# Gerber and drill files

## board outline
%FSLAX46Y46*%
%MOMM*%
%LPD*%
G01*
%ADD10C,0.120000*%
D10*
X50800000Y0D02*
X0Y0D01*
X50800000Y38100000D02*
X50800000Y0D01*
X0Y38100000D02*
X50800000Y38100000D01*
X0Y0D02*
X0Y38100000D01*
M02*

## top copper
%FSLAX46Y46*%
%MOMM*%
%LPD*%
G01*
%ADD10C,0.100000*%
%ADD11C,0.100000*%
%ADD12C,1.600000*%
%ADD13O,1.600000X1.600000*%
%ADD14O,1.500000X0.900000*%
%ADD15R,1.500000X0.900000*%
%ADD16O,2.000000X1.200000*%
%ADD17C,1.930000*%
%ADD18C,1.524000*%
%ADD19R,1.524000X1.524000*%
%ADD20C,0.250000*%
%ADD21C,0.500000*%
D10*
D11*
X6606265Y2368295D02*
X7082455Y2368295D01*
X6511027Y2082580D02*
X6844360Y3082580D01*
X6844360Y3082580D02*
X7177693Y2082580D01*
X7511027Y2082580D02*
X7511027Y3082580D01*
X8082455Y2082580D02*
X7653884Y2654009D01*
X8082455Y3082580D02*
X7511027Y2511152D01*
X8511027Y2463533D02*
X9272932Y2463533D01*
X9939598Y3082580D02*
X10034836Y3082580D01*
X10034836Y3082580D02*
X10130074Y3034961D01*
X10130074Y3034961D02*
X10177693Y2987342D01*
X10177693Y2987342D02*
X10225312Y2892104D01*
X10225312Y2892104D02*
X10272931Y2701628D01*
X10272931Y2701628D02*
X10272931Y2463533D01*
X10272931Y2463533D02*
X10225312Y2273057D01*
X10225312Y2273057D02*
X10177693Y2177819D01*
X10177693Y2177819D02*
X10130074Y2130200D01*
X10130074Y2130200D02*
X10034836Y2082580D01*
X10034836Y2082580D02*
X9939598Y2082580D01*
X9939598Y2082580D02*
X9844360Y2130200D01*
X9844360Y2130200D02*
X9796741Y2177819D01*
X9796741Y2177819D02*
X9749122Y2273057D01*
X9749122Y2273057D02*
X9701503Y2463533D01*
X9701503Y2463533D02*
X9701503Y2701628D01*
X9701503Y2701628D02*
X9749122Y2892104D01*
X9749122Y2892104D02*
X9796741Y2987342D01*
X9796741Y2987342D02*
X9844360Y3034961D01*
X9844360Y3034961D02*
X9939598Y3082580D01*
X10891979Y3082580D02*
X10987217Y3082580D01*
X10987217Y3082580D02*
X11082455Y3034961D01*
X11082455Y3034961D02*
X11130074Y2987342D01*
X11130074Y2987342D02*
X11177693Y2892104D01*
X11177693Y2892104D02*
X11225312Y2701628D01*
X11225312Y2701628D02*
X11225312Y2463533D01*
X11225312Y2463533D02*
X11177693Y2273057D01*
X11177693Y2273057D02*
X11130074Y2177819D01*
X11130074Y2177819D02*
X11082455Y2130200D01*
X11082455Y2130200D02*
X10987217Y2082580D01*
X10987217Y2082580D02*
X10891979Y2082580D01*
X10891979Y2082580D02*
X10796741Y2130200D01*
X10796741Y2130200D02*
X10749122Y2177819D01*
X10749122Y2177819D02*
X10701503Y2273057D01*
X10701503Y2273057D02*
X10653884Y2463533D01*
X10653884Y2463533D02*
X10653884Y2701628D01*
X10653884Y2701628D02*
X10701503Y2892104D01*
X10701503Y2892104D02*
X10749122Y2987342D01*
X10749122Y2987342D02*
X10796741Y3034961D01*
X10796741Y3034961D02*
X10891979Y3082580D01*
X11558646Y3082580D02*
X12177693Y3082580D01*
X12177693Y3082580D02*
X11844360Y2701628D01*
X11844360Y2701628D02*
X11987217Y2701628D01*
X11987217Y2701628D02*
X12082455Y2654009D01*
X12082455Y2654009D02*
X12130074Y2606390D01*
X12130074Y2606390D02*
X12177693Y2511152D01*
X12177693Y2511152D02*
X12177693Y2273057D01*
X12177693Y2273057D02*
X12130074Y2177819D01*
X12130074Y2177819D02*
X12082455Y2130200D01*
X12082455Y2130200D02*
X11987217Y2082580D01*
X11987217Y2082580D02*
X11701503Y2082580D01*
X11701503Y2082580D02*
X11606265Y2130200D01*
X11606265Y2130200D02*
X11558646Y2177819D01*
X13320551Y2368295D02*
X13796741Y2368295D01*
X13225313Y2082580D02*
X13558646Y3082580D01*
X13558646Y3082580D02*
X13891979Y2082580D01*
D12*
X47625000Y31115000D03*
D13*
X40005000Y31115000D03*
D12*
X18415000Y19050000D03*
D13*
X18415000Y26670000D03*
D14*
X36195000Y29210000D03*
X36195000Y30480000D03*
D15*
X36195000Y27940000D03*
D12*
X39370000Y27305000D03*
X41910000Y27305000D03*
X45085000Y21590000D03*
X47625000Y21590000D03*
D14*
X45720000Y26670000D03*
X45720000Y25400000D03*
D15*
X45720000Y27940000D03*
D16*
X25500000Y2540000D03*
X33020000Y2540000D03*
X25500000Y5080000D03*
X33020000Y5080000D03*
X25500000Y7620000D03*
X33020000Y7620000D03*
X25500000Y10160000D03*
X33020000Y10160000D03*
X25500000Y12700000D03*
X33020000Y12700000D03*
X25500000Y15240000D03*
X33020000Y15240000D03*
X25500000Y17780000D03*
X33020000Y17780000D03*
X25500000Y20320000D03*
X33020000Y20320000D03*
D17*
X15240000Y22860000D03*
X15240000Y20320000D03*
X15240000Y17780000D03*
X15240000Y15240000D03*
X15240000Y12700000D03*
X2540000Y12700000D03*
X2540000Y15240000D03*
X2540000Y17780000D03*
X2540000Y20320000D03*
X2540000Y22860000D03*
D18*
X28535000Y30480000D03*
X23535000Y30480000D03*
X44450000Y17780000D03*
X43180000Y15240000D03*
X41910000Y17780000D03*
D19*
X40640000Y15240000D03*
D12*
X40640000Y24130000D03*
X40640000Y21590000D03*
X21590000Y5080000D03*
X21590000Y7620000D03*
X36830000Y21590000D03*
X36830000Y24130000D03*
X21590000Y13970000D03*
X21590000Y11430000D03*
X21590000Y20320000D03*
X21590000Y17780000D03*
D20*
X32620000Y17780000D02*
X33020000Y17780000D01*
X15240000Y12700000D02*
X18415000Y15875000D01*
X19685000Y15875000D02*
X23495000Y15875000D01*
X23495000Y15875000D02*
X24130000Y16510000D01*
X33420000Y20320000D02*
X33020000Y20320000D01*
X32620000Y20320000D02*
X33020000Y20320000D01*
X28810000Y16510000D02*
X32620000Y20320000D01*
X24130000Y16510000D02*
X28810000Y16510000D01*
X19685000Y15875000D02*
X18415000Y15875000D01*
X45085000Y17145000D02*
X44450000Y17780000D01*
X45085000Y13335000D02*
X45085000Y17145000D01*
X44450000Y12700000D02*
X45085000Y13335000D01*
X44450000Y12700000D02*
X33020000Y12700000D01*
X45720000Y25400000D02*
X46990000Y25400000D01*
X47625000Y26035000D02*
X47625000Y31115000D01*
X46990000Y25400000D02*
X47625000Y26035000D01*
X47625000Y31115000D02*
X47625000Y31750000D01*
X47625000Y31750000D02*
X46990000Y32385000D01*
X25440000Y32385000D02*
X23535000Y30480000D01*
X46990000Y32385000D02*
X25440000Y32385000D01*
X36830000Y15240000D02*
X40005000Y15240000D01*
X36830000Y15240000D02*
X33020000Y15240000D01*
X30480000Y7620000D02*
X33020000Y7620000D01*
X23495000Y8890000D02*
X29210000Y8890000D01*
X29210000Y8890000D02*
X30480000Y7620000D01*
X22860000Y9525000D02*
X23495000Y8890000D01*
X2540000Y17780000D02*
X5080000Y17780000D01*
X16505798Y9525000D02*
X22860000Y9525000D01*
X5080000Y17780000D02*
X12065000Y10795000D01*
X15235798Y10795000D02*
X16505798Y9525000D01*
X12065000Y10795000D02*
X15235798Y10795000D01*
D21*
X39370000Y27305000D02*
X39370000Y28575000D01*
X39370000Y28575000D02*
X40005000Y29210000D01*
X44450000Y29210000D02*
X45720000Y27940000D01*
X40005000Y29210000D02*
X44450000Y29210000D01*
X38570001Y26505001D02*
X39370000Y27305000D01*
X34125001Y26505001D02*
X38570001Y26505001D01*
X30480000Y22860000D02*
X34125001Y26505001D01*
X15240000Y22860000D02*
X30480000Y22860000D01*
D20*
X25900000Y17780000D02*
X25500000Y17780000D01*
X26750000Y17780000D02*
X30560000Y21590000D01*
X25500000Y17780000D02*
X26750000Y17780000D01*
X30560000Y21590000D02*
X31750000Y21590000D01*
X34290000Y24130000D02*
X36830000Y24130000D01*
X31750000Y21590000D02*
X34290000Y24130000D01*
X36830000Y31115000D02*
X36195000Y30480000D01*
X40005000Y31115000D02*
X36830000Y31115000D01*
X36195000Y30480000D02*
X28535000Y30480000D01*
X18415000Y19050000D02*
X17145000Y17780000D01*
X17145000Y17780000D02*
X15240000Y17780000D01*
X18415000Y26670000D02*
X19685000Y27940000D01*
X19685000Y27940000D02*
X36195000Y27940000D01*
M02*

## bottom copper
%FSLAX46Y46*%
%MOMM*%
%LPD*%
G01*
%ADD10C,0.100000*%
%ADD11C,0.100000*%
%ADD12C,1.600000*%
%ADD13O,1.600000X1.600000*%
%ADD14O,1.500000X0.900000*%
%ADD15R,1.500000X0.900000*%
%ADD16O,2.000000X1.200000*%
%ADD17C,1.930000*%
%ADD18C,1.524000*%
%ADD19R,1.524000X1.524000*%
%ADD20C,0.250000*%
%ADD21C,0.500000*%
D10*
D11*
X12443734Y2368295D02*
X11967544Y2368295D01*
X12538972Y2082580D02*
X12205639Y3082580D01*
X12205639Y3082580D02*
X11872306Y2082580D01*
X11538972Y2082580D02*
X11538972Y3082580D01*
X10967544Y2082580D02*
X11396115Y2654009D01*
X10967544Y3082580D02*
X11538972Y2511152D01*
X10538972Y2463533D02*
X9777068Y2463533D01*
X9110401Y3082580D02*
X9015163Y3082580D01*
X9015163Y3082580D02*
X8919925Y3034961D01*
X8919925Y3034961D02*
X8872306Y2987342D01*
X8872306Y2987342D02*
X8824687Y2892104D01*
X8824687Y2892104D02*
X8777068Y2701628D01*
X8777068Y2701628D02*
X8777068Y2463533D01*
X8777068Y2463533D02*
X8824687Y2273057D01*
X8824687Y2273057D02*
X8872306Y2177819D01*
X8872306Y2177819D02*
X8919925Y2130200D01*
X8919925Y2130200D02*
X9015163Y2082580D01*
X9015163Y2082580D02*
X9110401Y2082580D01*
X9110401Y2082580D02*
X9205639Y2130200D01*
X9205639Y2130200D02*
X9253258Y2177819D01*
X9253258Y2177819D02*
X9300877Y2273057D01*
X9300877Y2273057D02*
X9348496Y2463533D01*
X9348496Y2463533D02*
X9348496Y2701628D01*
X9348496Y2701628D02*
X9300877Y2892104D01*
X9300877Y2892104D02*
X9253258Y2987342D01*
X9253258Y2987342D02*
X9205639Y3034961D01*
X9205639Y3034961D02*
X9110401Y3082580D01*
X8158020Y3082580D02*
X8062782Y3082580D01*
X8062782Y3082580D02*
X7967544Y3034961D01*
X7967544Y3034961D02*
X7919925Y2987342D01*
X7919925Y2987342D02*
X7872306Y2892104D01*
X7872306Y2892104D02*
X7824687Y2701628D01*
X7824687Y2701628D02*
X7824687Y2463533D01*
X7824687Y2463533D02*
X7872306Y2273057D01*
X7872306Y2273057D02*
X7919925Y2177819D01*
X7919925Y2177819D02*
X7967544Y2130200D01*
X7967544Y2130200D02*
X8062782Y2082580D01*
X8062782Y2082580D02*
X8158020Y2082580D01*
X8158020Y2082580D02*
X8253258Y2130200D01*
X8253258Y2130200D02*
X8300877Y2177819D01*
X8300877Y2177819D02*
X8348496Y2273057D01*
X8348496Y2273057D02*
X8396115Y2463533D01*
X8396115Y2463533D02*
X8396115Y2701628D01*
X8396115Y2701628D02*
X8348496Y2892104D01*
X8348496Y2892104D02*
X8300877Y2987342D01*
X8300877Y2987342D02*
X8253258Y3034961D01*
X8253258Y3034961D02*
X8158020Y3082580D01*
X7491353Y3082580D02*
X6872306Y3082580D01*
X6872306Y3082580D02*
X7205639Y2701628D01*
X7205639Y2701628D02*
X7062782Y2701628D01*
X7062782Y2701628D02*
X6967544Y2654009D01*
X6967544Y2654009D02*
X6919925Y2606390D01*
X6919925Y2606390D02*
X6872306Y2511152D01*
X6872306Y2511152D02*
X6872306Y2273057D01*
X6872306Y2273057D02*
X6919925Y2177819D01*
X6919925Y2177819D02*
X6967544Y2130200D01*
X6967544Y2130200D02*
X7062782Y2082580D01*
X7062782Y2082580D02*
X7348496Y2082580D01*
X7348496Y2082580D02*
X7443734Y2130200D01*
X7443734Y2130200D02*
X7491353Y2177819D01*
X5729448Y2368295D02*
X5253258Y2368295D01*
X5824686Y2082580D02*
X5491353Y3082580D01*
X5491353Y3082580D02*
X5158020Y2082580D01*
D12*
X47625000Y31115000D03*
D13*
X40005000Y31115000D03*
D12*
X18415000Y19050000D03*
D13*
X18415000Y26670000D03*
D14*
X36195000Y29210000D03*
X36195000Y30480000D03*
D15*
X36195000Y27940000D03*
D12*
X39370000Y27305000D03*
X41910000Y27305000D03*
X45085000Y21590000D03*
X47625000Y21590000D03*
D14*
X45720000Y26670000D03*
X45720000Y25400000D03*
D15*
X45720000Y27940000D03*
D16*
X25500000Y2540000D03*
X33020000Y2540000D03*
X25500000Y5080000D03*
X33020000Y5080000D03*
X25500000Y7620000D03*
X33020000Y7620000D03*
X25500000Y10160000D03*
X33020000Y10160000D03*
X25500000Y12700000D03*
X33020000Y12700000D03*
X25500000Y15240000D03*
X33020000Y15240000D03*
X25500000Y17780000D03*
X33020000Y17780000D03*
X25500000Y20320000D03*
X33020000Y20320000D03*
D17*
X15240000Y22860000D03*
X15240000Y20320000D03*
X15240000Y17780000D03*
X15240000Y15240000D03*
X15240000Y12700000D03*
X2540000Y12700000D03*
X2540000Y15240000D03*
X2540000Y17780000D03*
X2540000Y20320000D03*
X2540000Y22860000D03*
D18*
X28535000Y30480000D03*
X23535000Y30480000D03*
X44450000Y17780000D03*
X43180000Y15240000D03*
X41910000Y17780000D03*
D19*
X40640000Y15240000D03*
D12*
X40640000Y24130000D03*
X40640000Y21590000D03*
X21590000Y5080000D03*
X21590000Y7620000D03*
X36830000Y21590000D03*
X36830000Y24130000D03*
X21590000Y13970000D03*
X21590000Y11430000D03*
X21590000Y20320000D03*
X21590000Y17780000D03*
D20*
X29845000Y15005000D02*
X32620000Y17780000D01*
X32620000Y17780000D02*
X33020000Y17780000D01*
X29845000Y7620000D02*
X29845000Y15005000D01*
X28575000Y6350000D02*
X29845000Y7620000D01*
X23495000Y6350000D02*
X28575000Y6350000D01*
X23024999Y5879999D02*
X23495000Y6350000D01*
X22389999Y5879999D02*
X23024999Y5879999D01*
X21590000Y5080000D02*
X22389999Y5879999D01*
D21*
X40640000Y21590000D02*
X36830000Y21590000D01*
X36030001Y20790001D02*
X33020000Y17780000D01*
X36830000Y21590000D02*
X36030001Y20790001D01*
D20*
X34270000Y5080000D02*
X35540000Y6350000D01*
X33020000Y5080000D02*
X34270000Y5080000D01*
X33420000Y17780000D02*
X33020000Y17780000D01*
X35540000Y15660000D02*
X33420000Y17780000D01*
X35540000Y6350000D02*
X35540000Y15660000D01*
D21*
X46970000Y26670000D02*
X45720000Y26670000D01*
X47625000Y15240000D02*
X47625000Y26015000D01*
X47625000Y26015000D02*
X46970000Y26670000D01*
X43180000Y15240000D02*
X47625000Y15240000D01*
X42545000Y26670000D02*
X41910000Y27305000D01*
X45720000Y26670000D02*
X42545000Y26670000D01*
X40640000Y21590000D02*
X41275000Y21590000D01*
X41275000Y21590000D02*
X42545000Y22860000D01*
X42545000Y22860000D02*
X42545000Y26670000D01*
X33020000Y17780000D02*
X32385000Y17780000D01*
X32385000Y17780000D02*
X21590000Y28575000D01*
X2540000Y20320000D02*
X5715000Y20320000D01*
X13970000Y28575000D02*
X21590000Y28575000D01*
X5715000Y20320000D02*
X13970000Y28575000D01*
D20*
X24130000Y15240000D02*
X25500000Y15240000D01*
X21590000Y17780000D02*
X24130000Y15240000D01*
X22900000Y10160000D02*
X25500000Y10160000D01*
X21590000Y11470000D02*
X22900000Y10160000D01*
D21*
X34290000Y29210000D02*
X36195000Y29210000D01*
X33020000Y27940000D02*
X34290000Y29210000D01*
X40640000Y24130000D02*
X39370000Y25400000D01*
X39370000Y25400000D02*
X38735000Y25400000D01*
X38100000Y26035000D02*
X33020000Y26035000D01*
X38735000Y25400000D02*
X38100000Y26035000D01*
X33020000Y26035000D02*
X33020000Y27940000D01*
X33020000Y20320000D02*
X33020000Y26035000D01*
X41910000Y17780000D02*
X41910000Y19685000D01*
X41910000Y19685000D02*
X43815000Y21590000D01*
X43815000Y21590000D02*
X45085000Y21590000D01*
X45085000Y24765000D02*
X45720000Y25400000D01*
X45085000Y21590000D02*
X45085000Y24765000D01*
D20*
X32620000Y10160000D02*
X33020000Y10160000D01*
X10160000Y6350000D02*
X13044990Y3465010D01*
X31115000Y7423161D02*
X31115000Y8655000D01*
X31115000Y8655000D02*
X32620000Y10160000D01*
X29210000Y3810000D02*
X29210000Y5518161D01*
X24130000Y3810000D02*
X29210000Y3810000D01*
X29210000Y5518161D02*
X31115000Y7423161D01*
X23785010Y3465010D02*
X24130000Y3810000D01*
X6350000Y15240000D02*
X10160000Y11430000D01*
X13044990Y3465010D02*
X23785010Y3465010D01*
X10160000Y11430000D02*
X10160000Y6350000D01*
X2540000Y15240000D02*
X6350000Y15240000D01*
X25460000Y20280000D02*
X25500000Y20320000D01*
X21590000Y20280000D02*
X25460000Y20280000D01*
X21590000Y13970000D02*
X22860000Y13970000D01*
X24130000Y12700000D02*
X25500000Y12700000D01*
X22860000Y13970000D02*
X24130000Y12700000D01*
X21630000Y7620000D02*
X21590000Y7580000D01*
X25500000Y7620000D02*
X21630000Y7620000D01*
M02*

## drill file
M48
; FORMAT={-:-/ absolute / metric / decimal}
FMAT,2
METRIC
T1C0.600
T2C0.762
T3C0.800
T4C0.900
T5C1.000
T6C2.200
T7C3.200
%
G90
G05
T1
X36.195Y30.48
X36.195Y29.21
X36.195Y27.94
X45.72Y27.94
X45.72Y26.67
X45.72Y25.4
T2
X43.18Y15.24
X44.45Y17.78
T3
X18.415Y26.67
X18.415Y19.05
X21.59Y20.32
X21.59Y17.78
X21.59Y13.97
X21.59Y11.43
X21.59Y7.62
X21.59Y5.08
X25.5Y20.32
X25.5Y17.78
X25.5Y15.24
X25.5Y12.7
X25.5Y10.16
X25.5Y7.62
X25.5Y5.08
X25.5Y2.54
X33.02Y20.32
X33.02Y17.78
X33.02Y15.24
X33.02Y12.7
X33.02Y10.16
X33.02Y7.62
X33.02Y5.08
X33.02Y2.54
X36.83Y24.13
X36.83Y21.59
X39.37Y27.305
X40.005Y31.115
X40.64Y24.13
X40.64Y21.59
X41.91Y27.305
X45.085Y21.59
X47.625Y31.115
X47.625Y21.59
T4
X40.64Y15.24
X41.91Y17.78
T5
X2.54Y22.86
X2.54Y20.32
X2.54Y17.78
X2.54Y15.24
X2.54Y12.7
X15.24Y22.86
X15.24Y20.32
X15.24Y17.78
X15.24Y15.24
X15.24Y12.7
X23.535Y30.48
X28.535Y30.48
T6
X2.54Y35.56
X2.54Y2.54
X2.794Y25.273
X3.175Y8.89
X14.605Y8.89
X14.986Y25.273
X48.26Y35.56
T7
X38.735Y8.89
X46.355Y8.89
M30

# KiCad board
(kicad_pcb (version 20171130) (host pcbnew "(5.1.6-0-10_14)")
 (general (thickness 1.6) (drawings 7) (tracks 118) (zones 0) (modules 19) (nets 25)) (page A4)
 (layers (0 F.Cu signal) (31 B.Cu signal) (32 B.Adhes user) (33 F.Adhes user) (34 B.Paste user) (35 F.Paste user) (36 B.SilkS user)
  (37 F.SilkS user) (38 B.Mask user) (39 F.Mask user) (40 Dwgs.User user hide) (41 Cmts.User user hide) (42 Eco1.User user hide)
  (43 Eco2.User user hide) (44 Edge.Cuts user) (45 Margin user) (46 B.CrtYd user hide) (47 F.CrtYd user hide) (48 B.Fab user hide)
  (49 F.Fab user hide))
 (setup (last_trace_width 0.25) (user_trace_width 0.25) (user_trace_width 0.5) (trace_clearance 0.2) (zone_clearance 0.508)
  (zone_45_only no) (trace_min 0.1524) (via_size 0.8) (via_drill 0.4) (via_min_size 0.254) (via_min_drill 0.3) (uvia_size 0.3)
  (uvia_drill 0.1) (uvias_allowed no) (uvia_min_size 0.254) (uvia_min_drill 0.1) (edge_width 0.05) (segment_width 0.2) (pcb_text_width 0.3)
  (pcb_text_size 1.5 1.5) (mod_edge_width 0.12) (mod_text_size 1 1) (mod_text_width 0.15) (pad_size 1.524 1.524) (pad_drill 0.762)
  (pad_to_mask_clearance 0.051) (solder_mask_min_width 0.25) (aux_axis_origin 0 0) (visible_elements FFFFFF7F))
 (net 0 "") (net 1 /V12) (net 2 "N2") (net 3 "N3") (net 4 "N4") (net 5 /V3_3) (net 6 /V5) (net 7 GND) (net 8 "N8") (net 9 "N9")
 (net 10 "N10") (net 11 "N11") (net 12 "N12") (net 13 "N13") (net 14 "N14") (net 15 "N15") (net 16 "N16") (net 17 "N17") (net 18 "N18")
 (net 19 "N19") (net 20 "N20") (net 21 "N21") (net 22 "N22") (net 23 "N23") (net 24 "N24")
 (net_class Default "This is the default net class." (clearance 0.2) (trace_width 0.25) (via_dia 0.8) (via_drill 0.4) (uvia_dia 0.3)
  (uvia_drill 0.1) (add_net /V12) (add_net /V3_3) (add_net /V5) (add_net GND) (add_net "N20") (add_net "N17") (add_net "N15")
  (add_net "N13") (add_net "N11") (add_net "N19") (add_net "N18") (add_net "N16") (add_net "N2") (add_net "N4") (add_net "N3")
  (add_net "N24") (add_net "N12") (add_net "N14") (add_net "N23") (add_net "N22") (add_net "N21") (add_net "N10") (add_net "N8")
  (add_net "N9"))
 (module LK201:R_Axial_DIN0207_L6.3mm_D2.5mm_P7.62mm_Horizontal (layer F.Cu) (at 47.625 -31.115 180)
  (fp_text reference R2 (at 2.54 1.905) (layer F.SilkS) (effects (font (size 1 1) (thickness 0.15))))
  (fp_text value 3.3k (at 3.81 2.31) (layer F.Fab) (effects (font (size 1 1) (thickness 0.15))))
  (pad 1 thru_hole circle (at 0 0 180) (size 1.6 1.6) (drill 0.8) (layers *.Cu *.Mask) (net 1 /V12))
  (pad 2 thru_hole oval (at 7.62 0 180) (size 1.6 1.6) (drill 0.8) (layers *.Cu *.Mask) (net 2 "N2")))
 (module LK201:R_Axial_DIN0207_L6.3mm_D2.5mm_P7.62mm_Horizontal (layer F.Cu) (at 18.415 -19.05 90)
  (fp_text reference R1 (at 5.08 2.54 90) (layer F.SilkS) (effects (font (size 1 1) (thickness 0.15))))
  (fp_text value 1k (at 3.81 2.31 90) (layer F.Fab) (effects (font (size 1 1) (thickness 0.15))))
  (pad 1 thru_hole circle (at 0 0 90) (size 1.6 1.6) (drill 0.8) (layers *.Cu *.Mask) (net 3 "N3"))
  (pad 2 thru_hole oval (at 7.62 0 90) (size 1.6 1.6) (drill 0.8) (layers *.Cu *.Mask) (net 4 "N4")))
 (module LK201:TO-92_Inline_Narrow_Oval (layer F.Cu) (at 36.195 -27.94 90)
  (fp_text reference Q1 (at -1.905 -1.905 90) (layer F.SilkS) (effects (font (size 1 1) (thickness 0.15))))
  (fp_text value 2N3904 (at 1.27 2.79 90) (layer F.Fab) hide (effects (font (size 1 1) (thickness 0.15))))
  (pad 2 thru_hole oval (at 1.27 0 270) (size 0.9 1.5) (drill 0.6) (layers *.Cu *.Mask) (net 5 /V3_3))
  (pad 3 thru_hole oval (at 2.54 0 270) (size 0.9 1.5) (drill 0.6) (layers *.Cu *.Mask) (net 2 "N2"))
  (pad 1 thru_hole rect (at 0 0 270) (size 0.9 1.5) (drill 0.6) (layers *.Cu *.Mask) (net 4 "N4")))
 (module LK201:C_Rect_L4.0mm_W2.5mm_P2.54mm (layer F.Cu) (at 39.37 -27.305)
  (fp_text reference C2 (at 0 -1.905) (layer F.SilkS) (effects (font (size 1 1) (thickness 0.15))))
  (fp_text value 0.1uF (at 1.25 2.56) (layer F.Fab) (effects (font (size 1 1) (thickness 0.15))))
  (pad 1 thru_hole circle (at 0 0) (size 1.6 1.6) (drill 0.8) (layers *.Cu *.Mask) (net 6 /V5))
  (pad 2 thru_hole circle (at 2.54 0) (size 1.6 1.6) (drill 0.8) (layers *.Cu *.Mask) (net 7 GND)))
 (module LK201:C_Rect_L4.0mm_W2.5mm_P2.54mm (layer F.Cu) (at 45.085 -21.59)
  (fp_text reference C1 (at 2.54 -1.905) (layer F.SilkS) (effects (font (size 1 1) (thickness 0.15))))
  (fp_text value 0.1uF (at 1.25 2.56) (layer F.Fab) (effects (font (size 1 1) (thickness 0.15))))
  (pad 1 thru_hole circle (at 0 0) (size 1.6 1.6) (drill 0.8) (layers *.Cu *.Mask) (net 1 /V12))
  (pad 2 thru_hole circle (at 2.54 0) (size 1.6 1.6) (drill 0.8) (layers *.Cu *.Mask) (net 7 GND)))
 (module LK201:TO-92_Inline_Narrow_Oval (layer F.Cu) (at 45.72 -27.94 270)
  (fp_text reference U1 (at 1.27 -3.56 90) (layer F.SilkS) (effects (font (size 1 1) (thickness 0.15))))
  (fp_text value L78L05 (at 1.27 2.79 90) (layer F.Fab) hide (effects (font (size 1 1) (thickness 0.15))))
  (pad 2 thru_hole oval (at 1.27 0 90) (size 0.9 1.5) (drill 0.6) (layers *.Cu *.Mask) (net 7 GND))
  (pad 3 thru_hole oval (at 2.54 0 90) (size 0.9 1.5) (drill 0.6) (layers *.Cu *.Mask) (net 1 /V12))
  (pad 1 thru_hole rect (at 0 0 90) (size 0.9 1.5) (drill 0.6) (layers *.Cu *.Mask) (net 6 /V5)))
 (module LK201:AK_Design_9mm (layer F.Cu) (at 33.655 -33.655)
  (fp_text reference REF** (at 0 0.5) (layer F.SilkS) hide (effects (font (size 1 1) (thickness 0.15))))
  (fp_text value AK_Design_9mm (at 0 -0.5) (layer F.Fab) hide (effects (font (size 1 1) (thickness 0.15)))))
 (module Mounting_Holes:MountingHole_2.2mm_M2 (layer F.Cu) (at 2.54 -2.54)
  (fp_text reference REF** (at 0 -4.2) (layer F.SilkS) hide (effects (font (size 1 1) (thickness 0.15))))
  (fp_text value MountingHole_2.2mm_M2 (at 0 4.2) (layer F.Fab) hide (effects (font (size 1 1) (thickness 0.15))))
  (pad 1 np_thru_hole circle (at 0 0) (size 2.2 2.2) (drill 2.2) (layers *.Cu *.Mask)))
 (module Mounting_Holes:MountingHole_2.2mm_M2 (layer F.Cu) (at 2.54 -35.56)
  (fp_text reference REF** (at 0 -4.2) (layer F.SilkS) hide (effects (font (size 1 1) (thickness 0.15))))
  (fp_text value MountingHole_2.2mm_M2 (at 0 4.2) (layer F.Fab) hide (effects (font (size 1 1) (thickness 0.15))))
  (pad 1 np_thru_hole circle (at 0 0) (size 2.2 2.2) (drill 2.2) (layers *.Cu *.Mask)))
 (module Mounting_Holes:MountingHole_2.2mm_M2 (layer F.Cu) (at 48.26 -35.56)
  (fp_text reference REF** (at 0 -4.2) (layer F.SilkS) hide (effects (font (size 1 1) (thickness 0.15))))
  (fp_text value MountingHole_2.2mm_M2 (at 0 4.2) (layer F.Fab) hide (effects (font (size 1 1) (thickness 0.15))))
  (pad 1 np_thru_hole circle (at 0 0) (size 2.2 2.2) (drill 2.2) (layers *.Cu *.Mask)))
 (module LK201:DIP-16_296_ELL (layer F.Cu) (at 29.26 -11.43 270)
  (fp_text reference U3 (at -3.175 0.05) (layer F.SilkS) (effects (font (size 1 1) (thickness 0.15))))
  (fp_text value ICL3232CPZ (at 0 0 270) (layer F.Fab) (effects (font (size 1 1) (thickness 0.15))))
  (pad 8 thru_hole oval (at 8.89 3.76 270) (size 1.2 2) (drill 0.8) (layers *.Cu *.Mask) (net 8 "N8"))
  (pad 9 thru_hole oval (at 8.89 -3.76 270) (size 1.2 2) (drill 0.8) (layers *.Cu *.Mask) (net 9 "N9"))
  (pad 7 thru_hole oval (at 6.35 3.76 270) (size 1.2 2) (drill 0.8) (layers *.Cu *.Mask) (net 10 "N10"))
  (pad 10 thru_hole oval (at 6.35 -3.76 270) (size 1.2 2) (drill 0.8) (layers *.Cu *.Mask) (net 7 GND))
  (pad 6 thru_hole oval (at 3.81 3.76 270) (size 1.2 2) (drill 0.8) (layers *.Cu *.Mask) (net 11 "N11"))
  (pad 11 thru_hole oval (at 3.81 -3.76 270) (size 1.2 2) (drill 0.8) (layers *.Cu *.Mask) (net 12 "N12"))
  (pad 5 thru_hole oval (at 1.27 3.76 270) (size 1.2 2) (drill 0.8) (layers *.Cu *.Mask) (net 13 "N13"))
  (pad 12 thru_hole oval (at 1.27 -3.76 270) (size 1.2 2) (drill 0.8) (layers *.Cu *.Mask) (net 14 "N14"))
  (pad 4 thru_hole oval (at -1.27 3.76 270) (size 1.2 2) (drill 0.8) (layers *.Cu *.Mask) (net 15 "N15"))
  (pad 13 thru_hole oval (at -1.27 -3.76 270) (size 1.2 2) (drill 0.8) (layers *.Cu *.Mask) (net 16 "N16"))
  (pad 3 thru_hole oval (at -3.81 3.76 270) (size 1.2 2) (drill 0.8) (layers *.Cu *.Mask) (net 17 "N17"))
  (pad 14 thru_hole oval (at -3.81 -3.76 270) (size 1.2 2) (drill 0.8) (layers *.Cu *.Mask) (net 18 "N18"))
  (pad 2 thru_hole oval (at -6.35 3.76 270) (size 1.2 2) (drill 0.8) (layers *.Cu *.Mask) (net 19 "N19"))
  (pad 15 thru_hole oval (at -6.35 -3.76 270) (size 1.2 2) (drill 0.8) (layers *.Cu *.Mask) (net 7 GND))
  (pad 1 thru_hole oval (at -8.89 3.76 270) (size 1.2 2) (drill 0.8) (layers *.Cu *.Mask) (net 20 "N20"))
  (pad 16 thru_hole oval (at -8.89 -3.76 270) (size 1.2 2) (drill 0.8) (layers *.Cu *.Mask) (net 5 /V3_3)))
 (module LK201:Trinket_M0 (layer F.Cu) (at 8.89 -19.05 180)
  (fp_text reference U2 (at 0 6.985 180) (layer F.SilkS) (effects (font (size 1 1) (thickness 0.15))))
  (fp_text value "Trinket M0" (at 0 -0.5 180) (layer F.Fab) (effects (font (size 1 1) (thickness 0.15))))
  (pad 10 thru_hole circle (at -6.35 3.81 180) (size 1.93 1.93) (drill 1) (layers *.Cu *.Mask) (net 6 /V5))
  (pad 9 thru_hole circle (at -6.35 1.27 180) (size 1.93 1.93) (drill 1) (layers *.Cu *.Mask) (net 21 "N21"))
  (pad 8 thru_hole circle (at -6.35 -1.27 180) (size 1.93 1.93) (drill 1) (layers *.Cu *.Mask) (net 3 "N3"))
  (pad 7 thru_hole circle (at -6.35 -3.81 180) (size 1.93 1.93) (drill 1) (layers *.Cu *.Mask) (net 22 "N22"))
  (pad 6 thru_hole circle (at -6.35 -6.35 180) (size 1.93 1.93) (drill 1) (layers *.Cu *.Mask) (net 5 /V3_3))
  (pad 5 thru_hole circle (at 6.35 -6.35 180) (size 1.93 1.93) (drill 1) (layers *.Cu *.Mask) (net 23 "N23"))
  (pad 4 thru_hole circle (at 6.35 -3.81 180) (size 1.93 1.93) (drill 1) (layers *.Cu *.Mask) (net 14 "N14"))
  (pad 3 thru_hole circle (at 6.35 -1.27 180) (size 1.93 1.93) (drill 1) (layers *.Cu *.Mask) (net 12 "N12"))
  (pad 2 thru_hole circle (at 6.35 1.27 180) (size 1.93 1.93) (drill 1) (layers *.Cu *.Mask) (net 7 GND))
  (pad 1 thru_hole circle (at 6.35 3.81 180) (size 1.93 1.93) (drill 1) (layers *.Cu *.Mask) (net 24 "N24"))
  (pad "" np_thru_hole circle (at -5.715 -10.16 180) (size 2.2 2.2) (drill 2.2) (layers *.Mask F.Cu))
  (pad "" np_thru_hole circle (at 5.715 -10.16 180) (size 2.2 2.2) (drill 2.2) (layers *.Mask F.Cu))
  (pad "" np_thru_hole circle (at 6.096 6.223 180) (size 2.2 2.2) (drill 2.2) (layers *.Mask F.Cu))
  (pad "" np_thru_hole circle (at -6.096 6.223 180) (size 2.2 2.2) (drill 2.2) (layers *.Mask F.Cu)))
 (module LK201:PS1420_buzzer (layer F.Cu) (at 26.035 -30.48 180)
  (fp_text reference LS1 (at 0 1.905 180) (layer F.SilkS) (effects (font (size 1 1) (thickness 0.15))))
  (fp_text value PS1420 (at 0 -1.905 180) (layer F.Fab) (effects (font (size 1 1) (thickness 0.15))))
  (pad 2 thru_hole circle (at -2.5 0 180) (size 1.524 1.524) (drill 1) (layers *.Cu *.Mask) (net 2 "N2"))
  (pad 1 thru_hole circle (at 2.5 0 180) (size 1.524 1.524) (drill 1) (layers *.Cu *.Mask) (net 1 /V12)))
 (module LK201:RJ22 (layer F.Cu) (at 42.545 -8.89)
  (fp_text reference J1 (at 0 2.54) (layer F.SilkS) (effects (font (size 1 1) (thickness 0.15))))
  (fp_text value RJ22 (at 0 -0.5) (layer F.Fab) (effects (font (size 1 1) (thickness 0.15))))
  (pad "" np_thru_hole circle (at -3.81 0) (size 3.2 3.2) (drill 3.2) (layers *.Mask F.Cu))
  (pad "" np_thru_hole circle (at 3.81 0) (size 3.2 3.2) (drill 3.2) (layers *.Mask F.Cu))
  (pad 4 thru_hole circle (at 1.905 -8.89) (size 1.524 1.524) (drill 0.762) (layers *.Cu *.Mask) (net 16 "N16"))
  (pad 3 thru_hole circle (at 0.635 -6.35) (size 1.524 1.524) (drill 0.762) (layers *.Cu *.Mask) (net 7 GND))
  (pad 2 thru_hole circle (at -0.635 -8.89) (size 1.524 1.524) (drill 0.9) (layers *.Cu *.Mask) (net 1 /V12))
  (pad 1 thru_hole rect (at -1.905 -6.35) (size 1.524 1.524) (drill 0.9) (layers *.Cu *.Mask) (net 18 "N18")))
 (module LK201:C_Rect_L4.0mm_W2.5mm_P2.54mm (layer F.Cu) (at 40.64 -24.13 270)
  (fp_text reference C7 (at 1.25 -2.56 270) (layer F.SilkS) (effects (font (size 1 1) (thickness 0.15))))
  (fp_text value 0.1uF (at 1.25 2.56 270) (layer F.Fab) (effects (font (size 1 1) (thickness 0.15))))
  (pad 1 thru_hole circle (at 0 0 270) (size 1.6 1.6) (drill 0.8) (layers *.Cu *.Mask) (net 5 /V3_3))
  (pad 2 thru_hole circle (at 2.54 0 270) (size 1.6 1.6) (drill 0.8) (layers *.Cu *.Mask) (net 7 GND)))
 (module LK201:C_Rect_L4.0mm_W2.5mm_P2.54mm (layer F.Cu) (at 21.59 -5.08 90)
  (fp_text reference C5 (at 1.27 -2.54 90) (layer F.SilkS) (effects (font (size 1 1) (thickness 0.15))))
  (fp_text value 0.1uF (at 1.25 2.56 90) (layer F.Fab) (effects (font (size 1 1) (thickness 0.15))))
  (pad 1 thru_hole circle (at 0 0 90) (size 1.6 1.6) (drill 0.8) (layers *.Cu *.Mask) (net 7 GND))
  (pad 2 thru_hole circle (at 2.54 0 90) (size 1.6 1.6) (drill 0.8) (layers *.Cu *.Mask) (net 11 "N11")))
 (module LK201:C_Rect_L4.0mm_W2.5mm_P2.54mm (layer F.Cu) (at 36.83 -21.59 90)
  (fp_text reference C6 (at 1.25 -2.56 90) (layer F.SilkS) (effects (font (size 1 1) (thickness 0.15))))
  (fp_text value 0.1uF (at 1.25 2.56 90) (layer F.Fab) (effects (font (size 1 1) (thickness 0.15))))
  (pad 1 thru_hole circle (at 0 0 90) (size 1.6 1.6) (drill 0.8) (layers *.Cu *.Mask) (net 7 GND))
  (pad 2 thru_hole circle (at 2.54 0 90) (size 1.6 1.6) (drill 0.8) (layers *.Cu *.Mask) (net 19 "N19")))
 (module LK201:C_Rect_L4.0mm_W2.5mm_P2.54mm (layer F.Cu) (at 21.59 -13.97 270)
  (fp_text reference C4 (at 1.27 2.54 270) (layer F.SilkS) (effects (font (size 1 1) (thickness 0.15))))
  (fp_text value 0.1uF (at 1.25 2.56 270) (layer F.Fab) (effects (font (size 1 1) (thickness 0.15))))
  (pad 1 thru_hole circle (at 0 0 270) (size 1.6 1.6) (drill 0.8) (layers *.Cu *.Mask) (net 15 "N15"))
  (pad 2 thru_hole circle (at 2.54 0 270) (size 1.6 1.6) (drill 0.8) (layers *.Cu *.Mask) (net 13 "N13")))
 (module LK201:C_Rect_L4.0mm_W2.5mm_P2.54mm (layer F.Cu) (at 21.59 -20.32 270)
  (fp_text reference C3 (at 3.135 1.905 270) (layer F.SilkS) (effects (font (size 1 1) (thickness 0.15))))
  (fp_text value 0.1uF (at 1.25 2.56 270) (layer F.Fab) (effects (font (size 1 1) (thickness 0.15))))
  (pad 1 thru_hole circle (at 0 0 270) (size 1.6 1.6) (drill 0.8) (layers *.Cu *.Mask) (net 20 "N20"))
  (pad 2 thru_hole circle (at 2.54 0 270) (size 1.6 1.6) (drill 0.8) (layers *.Cu *.Mask) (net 17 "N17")))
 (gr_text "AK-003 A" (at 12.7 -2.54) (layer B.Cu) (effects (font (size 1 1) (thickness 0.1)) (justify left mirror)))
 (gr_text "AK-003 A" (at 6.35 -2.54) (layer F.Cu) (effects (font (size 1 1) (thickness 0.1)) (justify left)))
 (gr_line (start 50.8 0) (end 0 0) (layer Edge.Cuts) (width 0.12))
 (gr_line (start 50.8 -38.1) (end 50.8 0) (layer Edge.Cuts) (width 0.12))
 (gr_line (start 0 -38.1) (end 50.8 -38.1) (layer Edge.Cuts) (width 0.12))
 (gr_line (start 0 0) (end 0 -38.1) (layer Edge.Cuts) (width 0.12))
 (segment (start 29.845 -15.005) (end 32.62 -17.78) (width 0.25) (layer B.Cu) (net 7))
 (segment (start 32.62 -17.78) (end 33.02 -17.78) (width 0.25) (layer B.Cu) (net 7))
 (segment (start 29.845 -7.62) (end 29.845 -15.005) (width 0.25) (layer B.Cu) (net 7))
 (segment (start 28.575 -6.35) (end 29.845 -7.62) (width 0.25) (layer B.Cu) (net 7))
 (segment (start 23.495 -6.35) (end 28.575 -6.35) (width 0.25) (layer B.Cu) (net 7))
 (segment (start 23.024999 -5.879999) (end 23.495 -6.35) (width 0.25) (layer B.Cu) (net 7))
 (segment (start 22.389999 -5.879999) (end 23.024999 -5.879999) (width 0.25) (layer B.Cu) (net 7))
 (segment (start 21.59 -5.08) (end 22.389999 -5.879999) (width 0.25) (layer B.Cu) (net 7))
 (segment (start 32.62 -17.78) (end 33.02 -17.78) (width 0.25) (layer F.Cu) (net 7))
 (segment (start 40.64 -21.59) (end 36.83 -21.59) (width 0.5) (layer B.Cu) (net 7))
 (segment (start 36.030001 -20.790001) (end 33.02 -17.78) (width 0.5) (layer B.Cu) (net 7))
 (segment (start 36.83 -21.59) (end 36.030001 -20.790001) (width 0.5) (layer B.Cu) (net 7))
 (segment (start 34.27 -5.08) (end 35.54 -6.35) (width 0.25) (layer B.Cu) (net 7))
 (segment (start 33.02 -5.08) (end 34.27 -5.08) (width 0.25) (layer B.Cu) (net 7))
 (segment (start 33.42 -17.78) (end 33.02 -17.78) (width 0.25) (layer B.Cu) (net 7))
 (segment (start 35.54 -15.66) (end 33.42 -17.78) (width 0.25) (layer B.Cu) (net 7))
 (segment (start 35.54 -6.35) (end 35.54 -15.66) (width 0.25) (layer B.Cu) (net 7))
 (segment (start 46.97 -26.67) (end 45.72 -26.67) (width 0.5) (layer B.Cu) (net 7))
 (segment (start 47.625 -15.24) (end 47.625 -26.015) (width 0.5) (layer B.Cu) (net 7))
 (segment (start 47.625 -26.015) (end 46.97 -26.67) (width 0.5) (layer B.Cu) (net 7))
 (segment (start 43.18 -15.24) (end 47.625 -15.24) (width 0.5) (layer B.Cu) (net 7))
 (segment (start 42.545 -26.67) (end 41.91 -27.305) (width 0.5) (layer B.Cu) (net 7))
 (segment (start 45.72 -26.67) (end 42.545 -26.67) (width 0.5) (layer B.Cu) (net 7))
 (segment (start 40.64 -21.59) (end 41.275 -21.59) (width 0.5) (layer B.Cu) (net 7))
 (segment (start 41.275 -21.59) (end 42.545 -22.86) (width 0.5) (layer B.Cu) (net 7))
 (segment (start 42.545 -22.86) (end 42.545 -26.67) (width 0.5) (layer B.Cu) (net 7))
 (segment (start 33.02 -17.78) (end 32.385 -17.78) (width 0.5) (layer B.Cu) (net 7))
 (segment (start 32.385 -17.78) (end 21.59 -28.575) (width 0.5) (layer B.Cu) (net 7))
 (segment (start 2.54 -20.32) (end 5.715 -20.32) (width 0.5) (layer B.Cu) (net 7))
 (segment (start 13.97 -28.575) (end 21.59 -28.575) (width 0.5) (layer B.Cu) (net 7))
 (segment (start 5.715 -20.32) (end 13.97 -28.575) (width 0.5) (layer B.Cu) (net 7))
 (segment (start 24.13 -15.24) (end 25.5 -15.24) (width 0.25) (layer B.Cu) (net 17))
 (segment (start 21.59 -17.78) (end 24.13 -15.24) (width 0.25) (layer B.Cu) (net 17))
 (segment (start 22.9 -10.16) (end 25.5 -10.16) (width 0.25) (layer B.Cu) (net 13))
 (segment (start 21.59 -11.47) (end 22.9 -10.16) (width 0.25) (layer B.Cu) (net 13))
 (segment (start 15.24 -12.7) (end 18.415 -15.875) (width 0.25) (layer F.Cu) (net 5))
 (segment (start 19.685 -15.875) (end 23.495 -15.875) (width 0.25) (layer F.Cu) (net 5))
 (segment (start 23.495 -15.875) (end 24.13 -16.51) (width 0.25) (layer F.Cu) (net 5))
 (segment (start 33.42 -20.32) (end 33.02 -20.32) (width 0.25) (layer F.Cu) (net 5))
 (segment (start 32.62 -20.32) (end 33.02 -20.32) (width 0.25) (layer F.Cu) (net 5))
 (segment (start 28.81 -16.51) (end 32.62 -20.32) (width 0.25) (layer F.Cu) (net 5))
 (segment (start 24.13 -16.51) (end 28.81 -16.51) (width 0.25) (layer F.Cu) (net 5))
 (segment (start 34.29 -29.21) (end 36.195 -29.21) (width 0.5) (layer B.Cu) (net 5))
 (segment (start 33.02 -27.94) (end 34.29 -29.21) (width 0.5) (layer B.Cu) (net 5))
 (segment (start 40.64 -24.13) (end 39.37 -25.4) (width 0.5) (layer B.Cu) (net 5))
 (segment (start 39.37 -25.4) (end 38.735 -25.4) (width 0.5) (layer B.Cu) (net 5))
 (segment (start 38.1 -26.035) (end 33.02 -26.035) (width 0.5) (layer B.Cu) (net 5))
 (segment (start 38.735 -25.4) (end 38.1 -26.035) (width 0.5) (layer B.Cu) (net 5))
 (segment (start 33.02 -26.035) (end 33.02 -27.94) (width 0.5) (layer B.Cu) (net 5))
 (segment (start 33.02 -20.32) (end 33.02 -26.035) (width 0.5) (layer B.Cu) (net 5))
 (segment (start 19.685 -15.875) (end 18.415 -15.875) (width 0.25) (layer F.Cu) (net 5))
 (segment (start 45.085 -17.145) (end 44.45 -17.78) (width 0.25) (layer F.Cu) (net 16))
 (segment (start 45.085 -13.335) (end 45.085 -17.145) (width 0.25) (layer F.Cu) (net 16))
 (segment (start 44.45 -12.7) (end 45.085 -13.335) (width 0.25) (layer F.Cu) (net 16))
 (segment (start 44.45 -12.7) (end 33.02 -12.7) (width 0.25) (layer F.Cu) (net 16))
 (segment (start 41.91 -17.78) (end 41.91 -19.685) (width 0.5) (layer B.Cu) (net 1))
 (segment (start 41.91 -19.685) (end 43.815 -21.59) (width 0.5) (layer B.Cu) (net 1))
 (segment (start 43.815 -21.59) (end 45.085 -21.59) (width 0.5) (layer B.Cu) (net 1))
 (segment (start 45.085 -24.765) (end 45.72 -25.4) (width 0.5) (layer B.Cu) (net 1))
 (segment (start 45.085 -21.59) (end 45.085 -24.765) (width 0.5) (layer B.Cu) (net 1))
 (segment (start 45.72 -25.4) (end 46.99 -25.4) (width 0.25) (layer F.Cu) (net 1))
 (segment (start 47.625 -26.035) (end 47.625 -31.115) (width 0.25) (layer F.Cu) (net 1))
 (segment (start 46.99 -25.4) (end 47.625 -26.035) (width 0.25) (layer F.Cu) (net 1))
 (segment (start 47.625 -31.115) (end 47.625 -31.75) (width 0.25) (layer F.Cu) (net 1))
 (segment (start 47.625 -31.75) (end 46.99 -32.385) (width 0.25) (layer F.Cu) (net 1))
 (segment (start 25.44 -32.385) (end 23.535 -30.48) (width 0.25) (layer F.Cu) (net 1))
 (segment (start 46.99 -32.385) (end 25.44 -32.385) (width 0.25) (layer F.Cu) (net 1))
 (segment (start 36.83 -15.24) (end 40.005 -15.24) (width 0.25) (layer F.Cu) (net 18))
 (segment (start 36.83 -15.24) (end 33.02 -15.24) (width 0.25) (layer F.Cu) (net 18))
 (segment (start 32.62 -10.16) (end 33.02 -10.16) (width 0.25) (layer B.Cu) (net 14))
 (segment (start 10.16 -6.35) (end 13.04499 -3.46501) (width 0.25) (layer B.Cu) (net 14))
 (segment (start 31.115 -7.423161) (end 31.115 -8.655) (width 0.25) (layer B.Cu) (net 14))
 (segment (start 31.115 -8.655) (end 32.62 -10.16) (width 0.25) (layer B.Cu) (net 14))
 (segment (start 29.21 -3.81) (end 29.21 -5.518161) (width 0.25) (layer B.Cu) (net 14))
 (segment (start 24.13 -3.81) (end 29.21 -3.81) (width 0.25) (layer B.Cu) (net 14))
 (segment (start 29.21 -5.518161) (end 31.115 -7.423161) (width 0.25) (layer B.Cu) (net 14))
 (segment (start 23.78501 -3.46501) (end 24.13 -3.81) (width 0.25) (layer B.Cu) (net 14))
 (segment (start 6.35 -15.24) (end 10.16 -11.43) (width 0.25) (layer B.Cu) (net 14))
 (segment (start 13.04499 -3.46501) (end 23.78501 -3.46501) (width 0.25) (layer B.Cu) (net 14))
 (segment (start 10.16 -11.43) (end 10.16 -6.35) (width 0.25) (layer B.Cu) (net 14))
 (segment (start 2.54 -15.24) (end 6.35 -15.24) (width 0.25) (layer B.Cu) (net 14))
 (segment (start 30.48 -7.62) (end 33.02 -7.62) (width 0.25) (layer F.Cu) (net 12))
 (segment (start 23.495 -8.89) (end 29.21 -8.89) (width 0.25) (layer F.Cu) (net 12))
 (segment (start 29.21 -8.89) (end 30.48 -7.62) (width 0.25) (layer F.Cu) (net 12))
 (segment (start 22.86 -9.525) (end 23.495 -8.89) (width 0.25) (layer F.Cu) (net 12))
 (segment (start 2.54 -17.78) (end 5.08 -17.78) (width 0.25) (layer F.Cu) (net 12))
 (segment (start 16.505798 -9.525) (end 22.86 -9.525) (width 0.25) (layer F.Cu) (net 12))
 (segment (start 5.08 -17.78) (end 12.065 -10.795) (width 0.25) (layer F.Cu) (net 12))
 (segment (start 15.235798 -10.795) (end 16.505798 -9.525) (width 0.25) (layer F.Cu) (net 12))
 (segment (start 12.065 -10.795) (end 15.235798 -10.795) (width 0.25) (layer F.Cu) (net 12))
 (segment (start 39.37 -27.305) (end 39.37 -28.575) (width 0.5) (layer F.Cu) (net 6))
 (segment (start 39.37 -28.575) (end 40.005 -29.21) (width 0.5) (layer F.Cu) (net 6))
 (segment (start 44.45 -29.21) (end 45.72 -27.94) (width 0.5) (layer F.Cu) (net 6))
 (segment (start 40.005 -29.21) (end 44.45 -29.21) (width 0.5) (layer F.Cu) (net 6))
 (segment (start 38.570001 -26.505001) (end 39.37 -27.305) (width 0.5) (layer F.Cu) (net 6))
 (segment (start 34.125001 -26.505001) (end 38.570001 -26.505001) (width 0.5) (layer F.Cu) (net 6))
 (segment (start 30.48 -22.86) (end 34.125001 -26.505001) (width 0.5) (layer F.Cu) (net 6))
 (segment (start 15.24 -22.86) (end 30.48 -22.86) (width 0.5) (layer F.Cu) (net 6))
 (segment (start 25.46 -20.28) (end 25.5 -20.32) (width 0.25) (layer B.Cu) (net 20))
 (segment (start 21.59 -20.28) (end 25.46 -20.28) (width 0.25) (layer B.Cu) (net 20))
 (segment (start 21.59 -13.97) (end 22.86 -13.97) (width 0.25) (layer B.Cu) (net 15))
 (segment (start 24.13 -12.7) (end 25.5 -12.7) (width 0.25) (layer B.Cu) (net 15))
 (segment (start 22.86 -13.97) (end 24.13 -12.7) (width 0.25) (layer B.Cu) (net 15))
 (segment (start 21.63 -7.62) (end 21.59 -7.58) (width 0.25) (layer B.Cu) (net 11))
 (segment (start 25.5 -7.62) (end 21.63 -7.62) (width 0.25) (layer B.Cu) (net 11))
 (segment (start 25.9 -17.78) (end 25.5 -17.78) (width 0.25) (layer F.Cu) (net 19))
 (segment (start 26.75 -17.78) (end 30.56 -21.59) (width 0.25) (layer F.Cu) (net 19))
 (segment (start 25.5 -17.78) (end 26.75 -17.78) (width 0.25) (layer F.Cu) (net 19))
 (segment (start 30.56 -21.59) (end 31.75 -21.59) (width 0.25) (layer F.Cu) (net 19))
 (segment (start 34.29 -24.13) (end 36.83 -24.13) (width 0.25) (layer F.Cu) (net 19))
 (segment (start 31.75 -21.59) (end 34.29 -24.13) (width 0.25) (layer F.Cu) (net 19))
 (segment (start 36.83 -31.115) (end 36.195 -30.48) (width 0.25) (layer F.Cu) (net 2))
 (segment (start 40.005 -31.115) (end 36.83 -31.115) (width 0.25) (layer F.Cu) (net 2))
 (segment (start 36.195 -30.48) (end 28.535 -30.48) (width 0.25) (layer F.Cu) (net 2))
 (segment (start 18.415 -19.05) (end 17.145 -17.78) (width 0.25) (layer F.Cu) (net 3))
 (segment (start 17.145 -17.78) (end 15.24 -17.78) (width 0.25) (layer F.Cu) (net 3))
 (segment (start 18.415 -26.67) (end 19.685 -27.94) (width 0.25) (layer F.Cu) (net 4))
 (segment (start 19.685 -27.94) (end 36.195 -27.94) (width 0.25) (layer F.Cu) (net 4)))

